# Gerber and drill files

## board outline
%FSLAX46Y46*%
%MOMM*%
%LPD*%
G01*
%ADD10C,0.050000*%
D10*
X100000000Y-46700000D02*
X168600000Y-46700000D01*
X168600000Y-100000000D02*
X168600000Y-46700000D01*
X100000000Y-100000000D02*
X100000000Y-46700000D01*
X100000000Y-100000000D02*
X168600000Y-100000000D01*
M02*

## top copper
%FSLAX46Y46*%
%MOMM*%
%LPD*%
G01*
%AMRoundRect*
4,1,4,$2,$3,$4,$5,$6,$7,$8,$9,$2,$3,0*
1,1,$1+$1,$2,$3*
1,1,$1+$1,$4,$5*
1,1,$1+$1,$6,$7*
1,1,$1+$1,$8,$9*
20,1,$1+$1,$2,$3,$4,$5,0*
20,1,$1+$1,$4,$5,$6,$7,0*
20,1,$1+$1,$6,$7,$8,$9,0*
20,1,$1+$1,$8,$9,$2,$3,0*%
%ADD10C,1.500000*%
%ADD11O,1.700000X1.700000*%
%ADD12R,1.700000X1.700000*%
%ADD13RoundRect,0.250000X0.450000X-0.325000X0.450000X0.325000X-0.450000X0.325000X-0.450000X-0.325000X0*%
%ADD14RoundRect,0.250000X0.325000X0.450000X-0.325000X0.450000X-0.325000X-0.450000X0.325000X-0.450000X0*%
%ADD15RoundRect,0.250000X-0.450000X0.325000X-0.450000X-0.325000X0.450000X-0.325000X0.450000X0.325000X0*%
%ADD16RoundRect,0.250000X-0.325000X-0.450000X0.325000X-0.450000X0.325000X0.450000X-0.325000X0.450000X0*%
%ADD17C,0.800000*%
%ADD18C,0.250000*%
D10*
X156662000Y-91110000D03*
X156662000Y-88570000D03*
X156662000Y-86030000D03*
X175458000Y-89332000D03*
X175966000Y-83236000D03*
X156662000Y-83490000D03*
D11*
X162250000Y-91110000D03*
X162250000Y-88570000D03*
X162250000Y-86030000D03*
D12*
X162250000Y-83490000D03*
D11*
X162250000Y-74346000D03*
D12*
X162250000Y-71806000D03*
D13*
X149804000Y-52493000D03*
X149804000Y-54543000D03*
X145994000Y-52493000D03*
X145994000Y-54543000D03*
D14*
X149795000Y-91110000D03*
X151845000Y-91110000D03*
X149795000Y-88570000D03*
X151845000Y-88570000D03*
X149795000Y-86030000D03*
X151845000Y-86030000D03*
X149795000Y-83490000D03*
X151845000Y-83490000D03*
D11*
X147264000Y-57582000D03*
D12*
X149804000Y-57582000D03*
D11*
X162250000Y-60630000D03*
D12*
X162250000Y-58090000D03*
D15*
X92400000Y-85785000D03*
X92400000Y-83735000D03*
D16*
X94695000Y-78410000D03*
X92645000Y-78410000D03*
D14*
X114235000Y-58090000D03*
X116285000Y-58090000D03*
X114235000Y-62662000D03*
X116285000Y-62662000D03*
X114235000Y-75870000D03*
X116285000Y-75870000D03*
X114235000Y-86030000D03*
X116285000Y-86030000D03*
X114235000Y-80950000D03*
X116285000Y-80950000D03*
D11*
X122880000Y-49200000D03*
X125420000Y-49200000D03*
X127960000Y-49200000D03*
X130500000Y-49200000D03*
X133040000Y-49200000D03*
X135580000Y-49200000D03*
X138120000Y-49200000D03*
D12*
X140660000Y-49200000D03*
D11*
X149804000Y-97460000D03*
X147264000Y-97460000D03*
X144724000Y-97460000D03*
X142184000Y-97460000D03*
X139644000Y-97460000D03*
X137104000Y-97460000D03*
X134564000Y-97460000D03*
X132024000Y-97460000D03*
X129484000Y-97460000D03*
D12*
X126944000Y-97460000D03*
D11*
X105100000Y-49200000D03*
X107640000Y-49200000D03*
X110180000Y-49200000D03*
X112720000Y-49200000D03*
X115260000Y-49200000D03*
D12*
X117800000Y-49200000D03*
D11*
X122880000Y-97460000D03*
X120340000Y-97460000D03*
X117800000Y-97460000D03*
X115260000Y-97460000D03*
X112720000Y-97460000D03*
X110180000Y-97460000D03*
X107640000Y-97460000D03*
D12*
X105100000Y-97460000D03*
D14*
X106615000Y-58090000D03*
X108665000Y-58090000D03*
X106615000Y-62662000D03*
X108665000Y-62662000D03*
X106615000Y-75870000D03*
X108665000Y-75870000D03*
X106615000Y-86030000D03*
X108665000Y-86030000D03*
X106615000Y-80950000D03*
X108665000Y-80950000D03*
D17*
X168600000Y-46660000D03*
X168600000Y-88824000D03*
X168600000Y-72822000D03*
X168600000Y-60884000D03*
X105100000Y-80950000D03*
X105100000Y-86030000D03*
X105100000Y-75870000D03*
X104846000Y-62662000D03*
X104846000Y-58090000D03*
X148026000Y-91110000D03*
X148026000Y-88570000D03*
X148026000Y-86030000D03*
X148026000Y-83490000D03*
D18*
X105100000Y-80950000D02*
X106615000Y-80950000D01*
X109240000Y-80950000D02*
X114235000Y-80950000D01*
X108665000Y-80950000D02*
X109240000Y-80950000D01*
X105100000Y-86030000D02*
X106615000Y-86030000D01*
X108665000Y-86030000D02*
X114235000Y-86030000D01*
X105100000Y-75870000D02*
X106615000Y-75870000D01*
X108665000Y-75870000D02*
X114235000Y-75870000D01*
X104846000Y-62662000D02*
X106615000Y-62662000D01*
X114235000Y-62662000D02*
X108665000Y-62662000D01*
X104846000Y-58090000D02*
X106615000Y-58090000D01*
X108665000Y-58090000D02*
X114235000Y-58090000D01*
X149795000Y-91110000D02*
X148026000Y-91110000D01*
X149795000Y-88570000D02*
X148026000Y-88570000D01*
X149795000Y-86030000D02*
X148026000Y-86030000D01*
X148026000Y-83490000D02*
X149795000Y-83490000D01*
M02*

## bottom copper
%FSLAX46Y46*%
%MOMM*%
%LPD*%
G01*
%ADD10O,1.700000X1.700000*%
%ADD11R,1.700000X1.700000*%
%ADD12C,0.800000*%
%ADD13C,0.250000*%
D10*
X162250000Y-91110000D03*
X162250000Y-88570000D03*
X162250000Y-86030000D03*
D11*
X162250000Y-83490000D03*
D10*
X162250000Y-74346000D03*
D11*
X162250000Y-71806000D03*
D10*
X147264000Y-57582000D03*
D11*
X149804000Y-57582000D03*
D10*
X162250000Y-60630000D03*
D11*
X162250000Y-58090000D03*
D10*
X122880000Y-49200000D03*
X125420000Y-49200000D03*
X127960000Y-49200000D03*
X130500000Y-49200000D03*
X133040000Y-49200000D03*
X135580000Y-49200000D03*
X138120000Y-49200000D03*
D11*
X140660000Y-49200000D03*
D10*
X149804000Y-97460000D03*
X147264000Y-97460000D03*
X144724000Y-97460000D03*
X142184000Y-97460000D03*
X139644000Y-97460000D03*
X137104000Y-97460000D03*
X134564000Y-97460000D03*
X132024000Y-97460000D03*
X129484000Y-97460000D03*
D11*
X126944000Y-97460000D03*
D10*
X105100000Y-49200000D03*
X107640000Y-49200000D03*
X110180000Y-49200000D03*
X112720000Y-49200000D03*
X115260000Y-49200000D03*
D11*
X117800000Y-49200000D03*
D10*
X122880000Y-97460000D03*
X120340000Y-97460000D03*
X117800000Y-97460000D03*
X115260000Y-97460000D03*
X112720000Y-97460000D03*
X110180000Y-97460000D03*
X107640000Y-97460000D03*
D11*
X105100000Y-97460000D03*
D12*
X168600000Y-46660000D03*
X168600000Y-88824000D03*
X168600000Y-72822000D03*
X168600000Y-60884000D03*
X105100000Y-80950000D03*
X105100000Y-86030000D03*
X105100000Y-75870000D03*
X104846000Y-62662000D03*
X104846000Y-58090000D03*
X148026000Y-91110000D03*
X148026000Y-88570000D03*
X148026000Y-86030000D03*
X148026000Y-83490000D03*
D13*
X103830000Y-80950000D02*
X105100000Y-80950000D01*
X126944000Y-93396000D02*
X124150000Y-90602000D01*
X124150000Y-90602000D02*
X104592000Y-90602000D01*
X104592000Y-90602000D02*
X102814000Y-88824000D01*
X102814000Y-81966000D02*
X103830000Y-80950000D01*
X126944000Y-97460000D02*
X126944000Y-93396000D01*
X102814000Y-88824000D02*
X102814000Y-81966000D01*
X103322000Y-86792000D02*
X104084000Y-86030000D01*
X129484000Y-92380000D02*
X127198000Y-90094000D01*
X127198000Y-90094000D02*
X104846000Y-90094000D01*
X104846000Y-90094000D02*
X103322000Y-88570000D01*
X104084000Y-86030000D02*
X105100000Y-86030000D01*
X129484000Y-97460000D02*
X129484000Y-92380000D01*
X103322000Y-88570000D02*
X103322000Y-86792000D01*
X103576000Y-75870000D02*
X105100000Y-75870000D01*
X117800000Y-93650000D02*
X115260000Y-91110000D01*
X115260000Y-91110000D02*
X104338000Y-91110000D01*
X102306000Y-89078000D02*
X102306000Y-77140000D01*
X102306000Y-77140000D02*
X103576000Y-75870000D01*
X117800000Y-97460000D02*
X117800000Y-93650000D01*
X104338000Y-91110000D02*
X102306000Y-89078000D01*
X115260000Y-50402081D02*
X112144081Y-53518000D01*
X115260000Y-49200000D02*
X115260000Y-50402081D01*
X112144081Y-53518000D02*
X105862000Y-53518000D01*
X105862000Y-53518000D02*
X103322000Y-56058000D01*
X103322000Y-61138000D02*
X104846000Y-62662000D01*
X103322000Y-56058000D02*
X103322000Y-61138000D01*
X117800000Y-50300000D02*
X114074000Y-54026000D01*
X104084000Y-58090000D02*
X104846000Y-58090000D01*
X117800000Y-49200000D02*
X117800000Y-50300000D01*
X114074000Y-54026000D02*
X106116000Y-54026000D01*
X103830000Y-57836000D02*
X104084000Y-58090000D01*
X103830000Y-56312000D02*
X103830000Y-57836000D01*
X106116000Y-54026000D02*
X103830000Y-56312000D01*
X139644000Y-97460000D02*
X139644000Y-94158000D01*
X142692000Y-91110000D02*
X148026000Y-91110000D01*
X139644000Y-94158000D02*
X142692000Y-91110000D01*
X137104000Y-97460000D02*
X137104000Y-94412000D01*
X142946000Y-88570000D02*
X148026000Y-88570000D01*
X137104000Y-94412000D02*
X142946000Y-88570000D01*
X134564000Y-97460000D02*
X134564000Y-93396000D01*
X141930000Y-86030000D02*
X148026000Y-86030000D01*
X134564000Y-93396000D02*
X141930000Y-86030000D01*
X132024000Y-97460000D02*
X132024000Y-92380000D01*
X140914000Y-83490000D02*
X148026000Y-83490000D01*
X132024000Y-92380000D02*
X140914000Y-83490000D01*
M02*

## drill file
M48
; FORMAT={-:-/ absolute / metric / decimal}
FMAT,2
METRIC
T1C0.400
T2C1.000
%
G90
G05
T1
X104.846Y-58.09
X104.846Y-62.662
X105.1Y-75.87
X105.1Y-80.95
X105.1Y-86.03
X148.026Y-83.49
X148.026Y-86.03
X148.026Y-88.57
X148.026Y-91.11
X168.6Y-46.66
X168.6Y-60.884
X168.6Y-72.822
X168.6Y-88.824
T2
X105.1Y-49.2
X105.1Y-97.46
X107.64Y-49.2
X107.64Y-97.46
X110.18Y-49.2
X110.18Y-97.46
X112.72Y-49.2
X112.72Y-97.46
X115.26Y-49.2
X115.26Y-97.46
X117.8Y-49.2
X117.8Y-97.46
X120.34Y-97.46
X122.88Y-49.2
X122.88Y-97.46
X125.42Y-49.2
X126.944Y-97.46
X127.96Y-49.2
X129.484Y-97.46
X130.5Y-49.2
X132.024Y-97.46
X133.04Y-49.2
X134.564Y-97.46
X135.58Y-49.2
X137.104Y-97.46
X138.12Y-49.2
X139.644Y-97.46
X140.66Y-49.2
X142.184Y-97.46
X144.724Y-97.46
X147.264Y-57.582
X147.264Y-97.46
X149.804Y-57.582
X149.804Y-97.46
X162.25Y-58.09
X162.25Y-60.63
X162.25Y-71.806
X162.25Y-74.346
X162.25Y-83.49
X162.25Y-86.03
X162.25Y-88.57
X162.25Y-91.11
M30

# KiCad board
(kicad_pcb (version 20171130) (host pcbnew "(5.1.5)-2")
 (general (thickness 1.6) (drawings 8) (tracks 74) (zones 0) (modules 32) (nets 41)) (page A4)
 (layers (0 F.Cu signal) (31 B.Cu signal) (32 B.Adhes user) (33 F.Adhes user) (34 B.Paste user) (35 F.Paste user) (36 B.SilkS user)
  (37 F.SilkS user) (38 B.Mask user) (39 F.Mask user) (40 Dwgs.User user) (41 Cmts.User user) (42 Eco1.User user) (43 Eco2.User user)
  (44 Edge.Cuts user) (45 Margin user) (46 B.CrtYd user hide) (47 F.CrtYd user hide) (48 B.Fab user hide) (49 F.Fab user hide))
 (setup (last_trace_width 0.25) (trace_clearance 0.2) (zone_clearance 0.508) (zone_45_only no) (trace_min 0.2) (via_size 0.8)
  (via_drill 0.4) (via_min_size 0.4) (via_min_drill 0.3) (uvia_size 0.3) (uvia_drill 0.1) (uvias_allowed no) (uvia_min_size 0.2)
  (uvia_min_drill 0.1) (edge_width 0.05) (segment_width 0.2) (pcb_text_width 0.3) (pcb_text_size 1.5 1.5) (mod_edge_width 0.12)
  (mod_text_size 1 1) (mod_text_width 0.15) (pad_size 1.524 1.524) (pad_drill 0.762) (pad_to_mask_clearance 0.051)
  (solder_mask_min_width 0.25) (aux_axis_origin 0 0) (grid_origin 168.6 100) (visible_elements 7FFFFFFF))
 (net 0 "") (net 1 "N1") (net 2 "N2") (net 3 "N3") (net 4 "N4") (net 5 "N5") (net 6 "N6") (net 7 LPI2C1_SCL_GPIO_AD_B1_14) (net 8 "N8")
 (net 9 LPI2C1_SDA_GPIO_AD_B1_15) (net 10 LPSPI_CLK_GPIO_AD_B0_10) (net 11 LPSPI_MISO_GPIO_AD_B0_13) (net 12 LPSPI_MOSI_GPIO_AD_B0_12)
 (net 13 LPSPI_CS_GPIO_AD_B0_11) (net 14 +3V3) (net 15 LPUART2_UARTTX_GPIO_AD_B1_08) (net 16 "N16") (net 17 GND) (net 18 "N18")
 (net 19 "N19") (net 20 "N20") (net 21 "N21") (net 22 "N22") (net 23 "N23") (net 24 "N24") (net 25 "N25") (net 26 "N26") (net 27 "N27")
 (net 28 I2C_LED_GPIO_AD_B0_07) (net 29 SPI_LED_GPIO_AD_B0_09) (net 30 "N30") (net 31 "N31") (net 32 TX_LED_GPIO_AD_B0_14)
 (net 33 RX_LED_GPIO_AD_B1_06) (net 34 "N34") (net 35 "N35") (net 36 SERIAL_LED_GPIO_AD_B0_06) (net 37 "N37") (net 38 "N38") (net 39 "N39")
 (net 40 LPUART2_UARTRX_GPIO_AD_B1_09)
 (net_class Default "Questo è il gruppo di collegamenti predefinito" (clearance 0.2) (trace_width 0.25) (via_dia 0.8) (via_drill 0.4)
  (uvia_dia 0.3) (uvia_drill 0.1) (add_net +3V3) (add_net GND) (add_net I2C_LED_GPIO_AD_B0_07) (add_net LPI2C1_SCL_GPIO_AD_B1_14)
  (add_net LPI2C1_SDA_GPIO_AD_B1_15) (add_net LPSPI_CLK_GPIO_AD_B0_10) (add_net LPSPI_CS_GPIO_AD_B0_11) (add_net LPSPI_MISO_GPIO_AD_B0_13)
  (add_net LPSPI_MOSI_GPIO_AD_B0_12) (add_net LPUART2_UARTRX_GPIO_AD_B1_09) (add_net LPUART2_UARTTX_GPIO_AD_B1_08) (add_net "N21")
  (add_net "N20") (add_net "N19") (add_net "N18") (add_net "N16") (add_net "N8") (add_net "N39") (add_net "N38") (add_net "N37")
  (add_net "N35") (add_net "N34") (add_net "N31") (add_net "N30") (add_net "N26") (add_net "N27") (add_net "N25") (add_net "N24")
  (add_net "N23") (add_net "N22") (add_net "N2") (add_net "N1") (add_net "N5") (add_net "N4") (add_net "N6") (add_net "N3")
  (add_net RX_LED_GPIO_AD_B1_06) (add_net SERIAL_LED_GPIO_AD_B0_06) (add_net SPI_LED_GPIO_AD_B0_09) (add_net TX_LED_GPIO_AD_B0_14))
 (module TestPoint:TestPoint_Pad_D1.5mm (layer F.Cu) (at 156.662 91.11)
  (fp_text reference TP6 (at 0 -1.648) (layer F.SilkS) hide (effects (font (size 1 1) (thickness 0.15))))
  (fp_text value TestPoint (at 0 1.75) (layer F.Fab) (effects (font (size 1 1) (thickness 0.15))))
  (pad 1 smd circle (at 0 0) (size 1.5 1.5) (layers F.Cu F.Mask) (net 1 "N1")))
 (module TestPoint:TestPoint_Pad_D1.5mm (layer F.Cu) (at 156.662 88.57)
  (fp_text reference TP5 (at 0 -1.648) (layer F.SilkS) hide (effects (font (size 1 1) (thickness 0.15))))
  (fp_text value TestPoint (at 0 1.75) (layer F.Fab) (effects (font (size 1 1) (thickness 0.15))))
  (pad 1 smd circle (at 0 0) (size 1.5 1.5) (layers F.Cu F.Mask) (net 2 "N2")))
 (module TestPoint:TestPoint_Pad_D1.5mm (layer F.Cu) (at 156.662 86.03)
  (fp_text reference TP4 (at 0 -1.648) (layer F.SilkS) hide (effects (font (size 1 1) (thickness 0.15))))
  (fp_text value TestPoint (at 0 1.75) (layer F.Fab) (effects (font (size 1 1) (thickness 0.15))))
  (pad 1 smd circle (at 0 0) (size 1.5 1.5) (layers F.Cu F.Mask) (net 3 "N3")))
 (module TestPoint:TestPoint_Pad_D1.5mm (layer F.Cu) (at 175.458 89.332)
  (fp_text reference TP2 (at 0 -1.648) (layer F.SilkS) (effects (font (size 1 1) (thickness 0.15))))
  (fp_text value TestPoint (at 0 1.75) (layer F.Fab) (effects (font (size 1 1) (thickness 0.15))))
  (pad 1 smd circle (at 0 0) (size 1.5 1.5) (layers F.Cu F.Mask) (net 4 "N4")))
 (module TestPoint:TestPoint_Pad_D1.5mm (layer F.Cu) (at 175.966 83.236)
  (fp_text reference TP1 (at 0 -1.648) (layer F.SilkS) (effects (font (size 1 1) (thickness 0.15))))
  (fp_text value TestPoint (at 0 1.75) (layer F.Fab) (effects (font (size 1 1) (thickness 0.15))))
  (pad 1 smd circle (at 0 0) (size 1.5 1.5) (layers F.Cu F.Mask) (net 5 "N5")))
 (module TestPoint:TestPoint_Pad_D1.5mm (layer F.Cu) (at 156.662 83.49)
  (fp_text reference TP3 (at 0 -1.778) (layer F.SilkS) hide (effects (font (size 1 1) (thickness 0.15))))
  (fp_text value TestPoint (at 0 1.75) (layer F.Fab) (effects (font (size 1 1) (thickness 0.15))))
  (pad 1 smd circle (at 0 0) (size 1.5 1.5) (layers F.Cu F.Mask) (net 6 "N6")))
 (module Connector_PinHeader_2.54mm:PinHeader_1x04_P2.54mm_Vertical (layer F.Cu) (at 162.25 83.49)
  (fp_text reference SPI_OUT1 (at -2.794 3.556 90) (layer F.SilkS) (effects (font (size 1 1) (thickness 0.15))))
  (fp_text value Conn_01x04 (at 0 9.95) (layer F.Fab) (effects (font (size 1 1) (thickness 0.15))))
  (pad 4 thru_hole oval (at 0 7.62) (size 1.7 1.7) (drill 1) (layers *.Cu *.Mask) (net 1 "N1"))
  (pad 3 thru_hole oval (at 0 5.08) (size 1.7 1.7) (drill 1) (layers *.Cu *.Mask) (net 2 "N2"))
  (pad 2 thru_hole oval (at 0 2.54) (size 1.7 1.7) (drill 1) (layers *.Cu *.Mask) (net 3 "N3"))
  (pad 1 thru_hole rect (at 0 0) (size 1.7 1.7) (drill 1) (layers *.Cu *.Mask) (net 6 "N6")))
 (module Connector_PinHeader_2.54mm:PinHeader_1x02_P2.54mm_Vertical (layer F.Cu) (at 162.25 71.806)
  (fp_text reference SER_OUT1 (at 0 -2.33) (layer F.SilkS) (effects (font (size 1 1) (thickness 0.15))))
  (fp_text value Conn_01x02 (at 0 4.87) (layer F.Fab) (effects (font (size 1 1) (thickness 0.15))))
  (pad 2 thru_hole oval (at 0 2.54) (size 1.7 1.7) (drill 1) (layers *.Cu *.Mask) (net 4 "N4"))
  (pad 1 thru_hole rect (at 0 0) (size 1.7 1.7) (drill 1) (layers *.Cu *.Mask) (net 5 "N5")))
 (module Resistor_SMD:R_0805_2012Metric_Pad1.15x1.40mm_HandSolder (layer F.Cu) (at 149.804 53.518 90)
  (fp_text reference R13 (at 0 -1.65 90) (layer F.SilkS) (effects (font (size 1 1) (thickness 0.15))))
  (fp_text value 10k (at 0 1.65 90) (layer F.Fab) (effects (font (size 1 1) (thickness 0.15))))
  (pad 2 smd roundrect (at 1.025 0 90) (size 1.15 1.4) (layers F.Cu F.Paste F.Mask) (roundrect_rratio 0.217391)
   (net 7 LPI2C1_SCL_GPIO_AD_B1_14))
  (pad 1 smd roundrect (at -1.025 0 90) (size 1.15 1.4) (layers F.Cu F.Paste F.Mask) (roundrect_rratio 0.217391) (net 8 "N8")))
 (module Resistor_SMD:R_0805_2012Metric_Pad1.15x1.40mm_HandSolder (layer F.Cu) (at 145.994 53.518 90)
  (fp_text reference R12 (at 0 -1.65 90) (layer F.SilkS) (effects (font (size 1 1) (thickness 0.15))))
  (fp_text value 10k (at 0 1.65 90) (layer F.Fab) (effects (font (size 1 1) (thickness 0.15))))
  (pad 2 smd roundrect (at 1.025 0 90) (size 1.15 1.4) (layers F.Cu F.Paste F.Mask) (roundrect_rratio 0.217391)
   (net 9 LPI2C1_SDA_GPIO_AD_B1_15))
  (pad 1 smd roundrect (at -1.025 0 90) (size 1.15 1.4) (layers F.Cu F.Paste F.Mask) (roundrect_rratio 0.217391) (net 8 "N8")))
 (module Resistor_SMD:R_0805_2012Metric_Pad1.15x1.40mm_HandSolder (layer F.Cu) (at 150.82 91.11 180)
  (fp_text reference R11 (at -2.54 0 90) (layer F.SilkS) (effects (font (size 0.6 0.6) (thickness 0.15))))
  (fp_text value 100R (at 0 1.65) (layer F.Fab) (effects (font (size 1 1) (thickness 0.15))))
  (pad 2 smd roundrect (at 1.025 0 180) (size 1.15 1.4) (layers F.Cu F.Paste F.Mask) (roundrect_rratio 0.217391)
   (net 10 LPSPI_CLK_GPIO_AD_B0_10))
  (pad 1 smd roundrect (at -1.025 0 180) (size 1.15 1.4) (layers F.Cu F.Paste F.Mask) (roundrect_rratio 0.217391) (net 1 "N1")))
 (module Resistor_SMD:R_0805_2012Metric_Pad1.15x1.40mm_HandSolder (layer F.Cu) (at 150.82 88.57 180)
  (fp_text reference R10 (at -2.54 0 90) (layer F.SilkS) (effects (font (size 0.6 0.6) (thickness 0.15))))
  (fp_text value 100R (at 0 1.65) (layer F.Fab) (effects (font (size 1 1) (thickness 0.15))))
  (pad 2 smd roundrect (at 1.025 0 180) (size 1.15 1.4) (layers F.Cu F.Paste F.Mask) (roundrect_rratio 0.217391)
   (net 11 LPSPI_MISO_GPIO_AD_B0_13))
  (pad 1 smd roundrect (at -1.025 0 180) (size 1.15 1.4) (layers F.Cu F.Paste F.Mask) (roundrect_rratio 0.217391) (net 2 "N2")))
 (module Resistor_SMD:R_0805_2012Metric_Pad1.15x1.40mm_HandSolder (layer F.Cu) (at 150.82 86.03 180)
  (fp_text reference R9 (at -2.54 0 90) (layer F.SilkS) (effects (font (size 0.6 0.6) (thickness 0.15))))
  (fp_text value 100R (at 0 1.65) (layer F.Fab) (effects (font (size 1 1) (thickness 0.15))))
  (pad 2 smd roundrect (at 1.025 0 180) (size 1.15 1.4) (layers F.Cu F.Paste F.Mask) (roundrect_rratio 0.217391)
   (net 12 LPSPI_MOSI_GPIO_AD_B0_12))
  (pad 1 smd roundrect (at -1.025 0 180) (size 1.15 1.4) (layers F.Cu F.Paste F.Mask) (roundrect_rratio 0.217391) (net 3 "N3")))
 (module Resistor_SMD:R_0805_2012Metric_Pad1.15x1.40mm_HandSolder (layer F.Cu) (at 150.82 83.49 180)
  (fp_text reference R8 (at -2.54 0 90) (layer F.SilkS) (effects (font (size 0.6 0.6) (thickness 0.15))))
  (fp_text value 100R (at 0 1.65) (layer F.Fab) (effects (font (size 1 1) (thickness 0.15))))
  (pad 2 smd roundrect (at 1.025 0 180) (size 1.15 1.4) (layers F.Cu F.Paste F.Mask) (roundrect_rratio 0.217391)
   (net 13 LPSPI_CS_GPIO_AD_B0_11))
  (pad 1 smd roundrect (at -1.025 0 180) (size 1.15 1.4) (layers F.Cu F.Paste F.Mask) (roundrect_rratio 0.217391) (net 6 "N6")))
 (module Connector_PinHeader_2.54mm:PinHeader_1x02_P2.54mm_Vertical (layer F.Cu) (at 149.804 57.582 270)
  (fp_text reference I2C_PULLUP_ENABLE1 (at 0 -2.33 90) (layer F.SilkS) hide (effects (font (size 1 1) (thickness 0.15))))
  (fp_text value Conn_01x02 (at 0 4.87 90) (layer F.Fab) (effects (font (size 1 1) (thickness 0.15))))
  (pad 2 thru_hole oval (at 0 2.54 270) (size 1.7 1.7) (drill 1) (layers *.Cu *.Mask) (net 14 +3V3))
  (pad 1 thru_hole rect (at 0 0 270) (size 1.7 1.7) (drill 1) (layers *.Cu *.Mask) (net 8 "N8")))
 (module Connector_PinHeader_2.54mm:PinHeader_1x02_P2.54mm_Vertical (layer F.Cu) (at 162.25 58.09)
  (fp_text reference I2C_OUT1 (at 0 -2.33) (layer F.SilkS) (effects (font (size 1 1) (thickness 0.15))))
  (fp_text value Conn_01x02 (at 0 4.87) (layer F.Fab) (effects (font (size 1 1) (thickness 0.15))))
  (pad 2 thru_hole oval (at 0 2.54) (size 1.7 1.7) (drill 1) (layers *.Cu *.Mask) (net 7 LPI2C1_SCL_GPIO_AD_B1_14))
  (pad 1 thru_hole rect (at 0 0) (size 1.7 1.7) (drill 1) (layers *.Cu *.Mask) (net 9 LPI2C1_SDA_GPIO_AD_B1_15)))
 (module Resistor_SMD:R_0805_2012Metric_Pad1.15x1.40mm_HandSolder (layer F.Cu) (at 92.4 84.76 270)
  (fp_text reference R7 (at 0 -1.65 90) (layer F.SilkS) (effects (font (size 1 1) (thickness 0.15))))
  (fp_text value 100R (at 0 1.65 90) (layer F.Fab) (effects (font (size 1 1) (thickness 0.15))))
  (pad 2 smd roundrect (at 1.025 0 270) (size 1.15 1.4) (layers F.Cu F.Paste F.Mask) (roundrect_rratio 0.217391)
   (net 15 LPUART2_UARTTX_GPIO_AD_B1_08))
  (pad 1 smd roundrect (at -1.025 0 270) (size 1.15 1.4) (layers F.Cu F.Paste F.Mask) (roundrect_rratio 0.217391) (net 4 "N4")))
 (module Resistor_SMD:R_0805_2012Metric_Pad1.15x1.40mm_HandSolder (layer F.Cu) (at 93.67 78.41)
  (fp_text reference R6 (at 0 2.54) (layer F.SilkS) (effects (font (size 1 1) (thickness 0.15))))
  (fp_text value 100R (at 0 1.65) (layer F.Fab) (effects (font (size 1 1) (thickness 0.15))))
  (pad 2 smd roundrect (at 1.025 0) (size 1.15 1.4) (layers F.Cu F.Paste F.Mask) (roundrect_rratio 0.217391)
   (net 15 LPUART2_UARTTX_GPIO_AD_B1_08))
  (pad 1 smd roundrect (at -1.025 0) (size 1.15 1.4) (layers F.Cu F.Paste F.Mask) (roundrect_rratio 0.217391) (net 5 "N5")))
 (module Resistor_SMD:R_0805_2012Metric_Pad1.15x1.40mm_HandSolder (layer F.Cu) (at 115.26 58.09 180)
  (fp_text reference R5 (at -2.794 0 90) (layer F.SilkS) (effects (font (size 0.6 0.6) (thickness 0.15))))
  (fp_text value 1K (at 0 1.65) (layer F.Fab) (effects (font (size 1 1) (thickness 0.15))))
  (pad 2 smd roundrect (at 1.025 0 180) (size 1.15 1.4) (layers F.Cu F.Paste F.Mask) (roundrect_rratio 0.217391) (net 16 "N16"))
  (pad 1 smd roundrect (at -1.025 0 180) (size 1.15 1.4) (layers F.Cu F.Paste F.Mask) (roundrect_rratio 0.217391) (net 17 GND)))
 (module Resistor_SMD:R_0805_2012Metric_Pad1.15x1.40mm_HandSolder (layer F.Cu) (at 115.26 62.662 180)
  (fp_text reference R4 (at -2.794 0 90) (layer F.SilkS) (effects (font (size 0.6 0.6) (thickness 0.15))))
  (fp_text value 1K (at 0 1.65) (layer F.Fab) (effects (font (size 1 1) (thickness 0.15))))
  (pad 2 smd roundrect (at 1.025 0 180) (size 1.15 1.4) (layers F.Cu F.Paste F.Mask) (roundrect_rratio 0.217391) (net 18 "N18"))
  (pad 1 smd roundrect (at -1.025 0 180) (size 1.15 1.4) (layers F.Cu F.Paste F.Mask) (roundrect_rratio 0.217391) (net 17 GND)))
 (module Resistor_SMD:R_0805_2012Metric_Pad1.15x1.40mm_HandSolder (layer F.Cu) (at 115.26 75.87 180)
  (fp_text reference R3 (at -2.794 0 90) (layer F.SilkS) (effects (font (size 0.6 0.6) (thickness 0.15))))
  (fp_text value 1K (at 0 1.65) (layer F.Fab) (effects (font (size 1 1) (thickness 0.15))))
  (pad 2 smd roundrect (at 1.025 0 180) (size 1.15 1.4) (layers F.Cu F.Paste F.Mask) (roundrect_rratio 0.217391) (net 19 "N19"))
  (pad 1 smd roundrect (at -1.025 0 180) (size 1.15 1.4) (layers F.Cu F.Paste F.Mask) (roundrect_rratio 0.217391) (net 17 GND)))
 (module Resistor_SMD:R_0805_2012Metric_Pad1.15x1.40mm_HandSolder (layer F.Cu) (at 115.26 86.03 180)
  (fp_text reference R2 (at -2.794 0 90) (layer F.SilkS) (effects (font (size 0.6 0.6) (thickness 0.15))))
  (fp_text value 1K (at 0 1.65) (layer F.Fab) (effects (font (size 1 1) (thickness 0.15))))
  (pad 2 smd roundrect (at 1.025 0 180) (size 1.15 1.4) (layers F.Cu F.Paste F.Mask) (roundrect_rratio 0.217391) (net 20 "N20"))
  (pad 1 smd roundrect (at -1.025 0 180) (size 1.15 1.4) (layers F.Cu F.Paste F.Mask) (roundrect_rratio 0.217391) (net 17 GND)))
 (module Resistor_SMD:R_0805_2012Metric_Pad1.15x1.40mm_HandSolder (layer F.Cu) (at 115.26 80.95 180)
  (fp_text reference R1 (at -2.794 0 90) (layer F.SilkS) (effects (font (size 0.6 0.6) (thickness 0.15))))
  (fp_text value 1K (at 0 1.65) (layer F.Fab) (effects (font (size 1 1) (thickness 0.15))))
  (pad 2 smd roundrect (at 1.025 0 180) (size 1.15 1.4) (layers F.Cu F.Paste F.Mask) (roundrect_rratio 0.217391) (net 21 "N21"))
  (pad 1 smd roundrect (at -1.025 0 180) (size 1.15 1.4) (layers F.Cu F.Paste F.Mask) (roundrect_rratio 0.217391) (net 17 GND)))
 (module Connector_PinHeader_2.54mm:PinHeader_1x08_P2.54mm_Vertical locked (layer F.Cu) (at 140.66 49.2 270)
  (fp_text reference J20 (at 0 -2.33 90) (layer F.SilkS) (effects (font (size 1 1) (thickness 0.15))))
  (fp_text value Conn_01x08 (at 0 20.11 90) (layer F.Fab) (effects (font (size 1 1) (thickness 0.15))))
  (pad 8 thru_hole oval (at 0 17.78 270) (size 1.7 1.7) (drill 1) (layers *.Cu *.Mask) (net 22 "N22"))
  (pad 7 thru_hole oval (at 0 15.24 270) (size 1.7 1.7) (drill 1) (layers *.Cu *.Mask) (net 17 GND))
  (pad 6 thru_hole oval (at 0 12.7 270) (size 1.7 1.7) (drill 1) (layers *.Cu *.Mask) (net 17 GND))
  (pad 5 thru_hole oval (at 0 10.16 270) (size 1.7 1.7) (drill 1) (layers *.Cu *.Mask) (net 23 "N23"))
  (pad 4 thru_hole oval (at 0 7.62 270) (size 1.7 1.7) (drill 1) (layers *.Cu *.Mask) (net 14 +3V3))
  (pad 3 thru_hole oval (at 0 5.08 270) (size 1.7 1.7) (drill 1) (layers *.Cu *.Mask) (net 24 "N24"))
  (pad 2 thru_hole oval (at 0 2.54 270) (size 1.7 1.7) (drill 1) (layers *.Cu *.Mask) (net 14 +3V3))
  (pad 1 thru_hole rect (at 0 0 270) (size 1.7 1.7) (drill 1) (layers *.Cu *.Mask) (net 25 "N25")))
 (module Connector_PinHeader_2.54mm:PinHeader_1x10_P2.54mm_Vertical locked (layer F.Cu) (at 126.944 97.46 90)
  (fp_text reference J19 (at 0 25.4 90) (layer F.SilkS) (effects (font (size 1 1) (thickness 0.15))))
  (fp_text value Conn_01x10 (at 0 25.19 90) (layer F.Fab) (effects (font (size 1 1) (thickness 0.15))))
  (pad 10 thru_hole oval (at 0 22.86 90) (size 1.7 1.7) (drill 1) (layers *.Cu *.Mask) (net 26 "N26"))
  (pad 9 thru_hole oval (at 0 20.32 90) (size 1.7 1.7) (drill 1) (layers *.Cu *.Mask) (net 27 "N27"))
  (pad 8 thru_hole oval (at 0 17.78 90) (size 1.7 1.7) (drill 1) (layers *.Cu *.Mask) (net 14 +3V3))
  (pad 7 thru_hole oval (at 0 15.24 90) (size 1.7 1.7) (drill 1) (layers *.Cu *.Mask) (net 17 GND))
  (pad 6 thru_hole oval (at 0 12.7 90) (size 1.7 1.7) (drill 1) (layers *.Cu *.Mask) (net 10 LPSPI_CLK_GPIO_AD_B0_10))
  (pad 5 thru_hole oval (at 0 10.16 90) (size 1.7 1.7) (drill 1) (layers *.Cu *.Mask) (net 11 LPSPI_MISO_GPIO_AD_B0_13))
  (pad 4 thru_hole oval (at 0 7.62 90) (size 1.7 1.7) (drill 1) (layers *.Cu *.Mask) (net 12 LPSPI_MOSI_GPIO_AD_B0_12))
  (pad 3 thru_hole oval (at 0 5.08 90) (size 1.7 1.7) (drill 1) (layers *.Cu *.Mask) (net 13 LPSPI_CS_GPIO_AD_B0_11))
  (pad 2 thru_hole oval (at 0 2.54 90) (size 1.7 1.7) (drill 1) (layers *.Cu *.Mask) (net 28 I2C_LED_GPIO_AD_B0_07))
  (pad 1 thru_hole rect (at 0 0 90) (size 1.7 1.7) (drill 1) (layers *.Cu *.Mask) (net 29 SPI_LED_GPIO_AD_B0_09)))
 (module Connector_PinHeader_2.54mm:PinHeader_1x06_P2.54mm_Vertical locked (layer F.Cu) (at 117.8 49.2 270)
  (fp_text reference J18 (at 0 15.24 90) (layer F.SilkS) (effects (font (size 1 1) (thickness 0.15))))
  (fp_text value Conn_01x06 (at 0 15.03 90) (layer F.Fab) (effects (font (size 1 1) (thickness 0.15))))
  (pad 6 thru_hole oval (at 0 12.7 270) (size 1.7 1.7) (drill 1) (layers *.Cu *.Mask) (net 7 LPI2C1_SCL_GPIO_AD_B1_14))
  (pad 5 thru_hole oval (at 0 10.16 270) (size 1.7 1.7) (drill 1) (layers *.Cu *.Mask) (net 9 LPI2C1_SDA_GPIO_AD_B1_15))
  (pad 4 thru_hole oval (at 0 7.62 270) (size 1.7 1.7) (drill 1) (layers *.Cu *.Mask) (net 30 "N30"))
  (pad 3 thru_hole oval (at 0 5.08 270) (size 1.7 1.7) (drill 1) (layers *.Cu *.Mask) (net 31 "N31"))
  (pad 2 thru_hole oval (at 0 2.54 270) (size 1.7 1.7) (drill 1) (layers *.Cu *.Mask) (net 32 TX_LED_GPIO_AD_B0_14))
  (pad 1 thru_hole rect (at 0 0 270) (size 1.7 1.7) (drill 1) (layers *.Cu *.Mask) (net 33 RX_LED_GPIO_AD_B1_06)))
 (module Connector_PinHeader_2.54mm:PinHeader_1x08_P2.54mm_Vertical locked (layer F.Cu) (at 105.1 97.46 90)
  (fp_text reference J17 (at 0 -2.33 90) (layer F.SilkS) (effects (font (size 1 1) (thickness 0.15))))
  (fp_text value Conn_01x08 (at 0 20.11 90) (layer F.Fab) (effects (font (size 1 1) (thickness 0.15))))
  (pad 8 thru_hole oval (at 0 17.78 90) (size 1.7 1.7) (drill 1) (layers *.Cu *.Mask) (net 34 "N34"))
  (pad 7 thru_hole oval (at 0 15.24 90) (size 1.7 1.7) (drill 1) (layers *.Cu *.Mask) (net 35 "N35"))
  (pad 6 thru_hole oval (at 0 12.7 90) (size 1.7 1.7) (drill 1) (layers *.Cu *.Mask) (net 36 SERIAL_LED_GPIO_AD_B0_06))
  (pad 5 thru_hole oval (at 0 10.16 90) (size 1.7 1.7) (drill 1) (layers *.Cu *.Mask) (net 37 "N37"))
  (pad 4 thru_hole oval (at 0 7.62 90) (size 1.7 1.7) (drill 1) (layers *.Cu *.Mask) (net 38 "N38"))
  (pad 3 thru_hole oval (at 0 5.08 90) (size 1.7 1.7) (drill 1) (layers *.Cu *.Mask) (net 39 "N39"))
  (pad 2 thru_hole oval (at 0 2.54 90) (size 1.7 1.7) (drill 1) (layers *.Cu *.Mask) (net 15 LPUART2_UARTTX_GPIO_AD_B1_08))
  (pad 1 thru_hole rect (at 0 0 90) (size 1.7 1.7) (drill 1) (layers *.Cu *.Mask) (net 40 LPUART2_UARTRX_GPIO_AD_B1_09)))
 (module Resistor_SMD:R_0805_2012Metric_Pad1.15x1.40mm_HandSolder (layer F.Cu) (at 107.64 58.09 180)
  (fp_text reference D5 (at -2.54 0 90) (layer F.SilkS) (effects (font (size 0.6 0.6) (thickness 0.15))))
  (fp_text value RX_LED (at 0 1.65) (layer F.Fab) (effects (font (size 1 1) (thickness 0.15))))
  (pad 2 smd roundrect (at 1.025 0 180) (size 1.15 1.4) (layers F.Cu F.Paste F.Mask) (roundrect_rratio 0.217391)
   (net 33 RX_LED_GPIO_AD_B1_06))
  (pad 1 smd roundrect (at -1.025 0 180) (size 1.15 1.4) (layers F.Cu F.Paste F.Mask) (roundrect_rratio 0.217391) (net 16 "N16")))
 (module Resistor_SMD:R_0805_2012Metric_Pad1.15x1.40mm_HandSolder (layer F.Cu) (at 107.64 62.662 180)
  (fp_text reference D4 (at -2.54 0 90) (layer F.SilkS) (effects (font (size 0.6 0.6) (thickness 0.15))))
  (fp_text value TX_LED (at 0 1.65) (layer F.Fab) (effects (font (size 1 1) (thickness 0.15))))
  (pad 2 smd roundrect (at 1.025 0 180) (size 1.15 1.4) (layers F.Cu F.Paste F.Mask) (roundrect_rratio 0.217391)
   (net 32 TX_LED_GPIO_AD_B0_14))
  (pad 1 smd roundrect (at -1.025 0 180) (size 1.15 1.4) (layers F.Cu F.Paste F.Mask) (roundrect_rratio 0.217391) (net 18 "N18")))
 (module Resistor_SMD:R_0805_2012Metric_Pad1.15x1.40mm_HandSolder (layer F.Cu) (at 107.64 75.87 180)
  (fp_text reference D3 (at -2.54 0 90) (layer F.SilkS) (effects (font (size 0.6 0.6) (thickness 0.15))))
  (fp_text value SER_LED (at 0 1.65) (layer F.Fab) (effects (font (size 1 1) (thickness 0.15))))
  (pad 2 smd roundrect (at 1.025 0 180) (size 1.15 1.4) (layers F.Cu F.Paste F.Mask) (roundrect_rratio 0.217391)
   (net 36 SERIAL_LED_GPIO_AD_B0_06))
  (pad 1 smd roundrect (at -1.025 0 180) (size 1.15 1.4) (layers F.Cu F.Paste F.Mask) (roundrect_rratio 0.217391) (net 19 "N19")))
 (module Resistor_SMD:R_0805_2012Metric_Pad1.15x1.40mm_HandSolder (layer F.Cu) (at 107.64 86.03 180)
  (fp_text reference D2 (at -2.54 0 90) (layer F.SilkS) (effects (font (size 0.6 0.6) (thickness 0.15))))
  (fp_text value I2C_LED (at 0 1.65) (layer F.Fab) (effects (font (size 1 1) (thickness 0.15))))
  (pad 2 smd roundrect (at 1.025 0 180) (size 1.15 1.4) (layers F.Cu F.Paste F.Mask) (roundrect_rratio 0.217391)
   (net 28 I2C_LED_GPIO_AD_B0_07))
  (pad 1 smd roundrect (at -1.025 0 180) (size 1.15 1.4) (layers F.Cu F.Paste F.Mask) (roundrect_rratio 0.217391) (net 20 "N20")))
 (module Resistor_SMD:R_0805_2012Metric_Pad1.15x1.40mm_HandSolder (layer F.Cu) (at 107.64 80.95 180)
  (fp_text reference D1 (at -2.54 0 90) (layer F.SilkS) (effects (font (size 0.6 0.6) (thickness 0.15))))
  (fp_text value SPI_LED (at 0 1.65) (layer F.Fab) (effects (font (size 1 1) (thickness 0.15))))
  (pad 2 smd roundrect (at 1.025 0 180) (size 1.15 1.4) (layers F.Cu F.Paste F.Mask) (roundrect_rratio 0.217391)
   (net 29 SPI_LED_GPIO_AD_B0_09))
  (pad 1 smd roundrect (at -1.025 0 180) (size 1.15 1.4) (layers F.Cu F.Paste F.Mask) (roundrect_rratio 0.217391) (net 21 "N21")))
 (gr_line (start 100 46.7) (end 168.6 46.7) (layer Edge.Cuts) (width 0.05))
 (gr_line (start 168.6 100) (end 168.6 46.7) (layer Edge.Cuts) (width 0.05))
 (gr_line (start 100 100) (end 100 46.7) (layer Edge.Cuts) (width 0.05))
 (gr_line (start 100 100) (end 168.6 100) (layer Edge.Cuts) (width 0.05))
 (via (at 168.6 46.66) (size 0.8) (drill 0.4) (layers F.Cu B.Cu) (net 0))
 (via (at 168.6 88.824) (size 0.8) (drill 0.4) (layers F.Cu B.Cu) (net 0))
 (via (at 168.6 72.822) (size 0.8) (drill 0.4) (layers F.Cu B.Cu) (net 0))
 (via (at 168.6 60.884) (size 0.8) (drill 0.4) (layers F.Cu B.Cu) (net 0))
 (via (at 105.1 80.95) (size 0.8) (drill 0.4) (layers F.Cu B.Cu) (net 29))
 (segment (start 103.83 80.95) (end 105.1 80.95) (width 0.25) (layer B.Cu) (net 29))
 (segment (start 126.944 93.396) (end 124.15 90.602) (width 0.25) (layer B.Cu) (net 29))
 (segment (start 124.15 90.602) (end 104.592 90.602) (width 0.25) (layer B.Cu) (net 29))
 (segment (start 104.592 90.602) (end 102.814 88.824) (width 0.25) (layer B.Cu) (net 29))
 (segment (start 102.814 81.966) (end 103.83 80.95) (width 0.25) (layer B.Cu) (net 29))
 (segment (start 126.944 97.46) (end 126.944 93.396) (width 0.25) (layer B.Cu) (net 29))
 (segment (start 102.814 88.824) (end 102.814 81.966) (width 0.25) (layer B.Cu) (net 29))
 (segment (start 105.1 80.95) (end 106.615 80.95) (width 0.25) (layer F.Cu) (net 29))
 (segment (start 109.24 80.95) (end 114.235 80.95) (width 0.25) (layer F.Cu) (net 21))
 (segment (start 108.665 80.95) (end 109.24 80.95) (width 0.25) (layer F.Cu) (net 21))
 (via (at 105.1 86.03) (size 0.8) (drill 0.4) (layers F.Cu B.Cu) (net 28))
 (segment (start 103.322 86.792) (end 104.084 86.03) (width 0.25) (layer B.Cu) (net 28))
 (segment (start 129.484 92.38) (end 127.198 90.094) (width 0.25) (layer B.Cu) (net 28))
 (segment (start 127.198 90.094) (end 104.846 90.094) (width 0.25) (layer B.Cu) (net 28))
 (segment (start 104.846 90.094) (end 103.322 88.57) (width 0.25) (layer B.Cu) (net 28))
 (segment (start 104.084 86.03) (end 105.1 86.03) (width 0.25) (layer B.Cu) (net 28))
 (segment (start 129.484 97.46) (end 129.484 92.38) (width 0.25) (layer B.Cu) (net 28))
 (segment (start 103.322 88.57) (end 103.322 86.792) (width 0.25) (layer B.Cu) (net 28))
 (segment (start 105.1 86.03) (end 106.615 86.03) (width 0.25) (layer F.Cu) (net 28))
 (segment (start 108.665 86.03) (end 114.235 86.03) (width 0.25) (layer F.Cu) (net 20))
 (via (at 105.1 75.87) (size 0.8) (drill 0.4) (layers F.Cu B.Cu) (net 36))
 (segment (start 103.576 75.87) (end 105.1 75.87) (width 0.25) (layer B.Cu) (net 36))
 (segment (start 117.8 93.65) (end 115.26 91.11) (width 0.25) (layer B.Cu) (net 36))
 (segment (start 115.26 91.11) (end 104.338 91.11) (width 0.25) (layer B.Cu) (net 36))
 (segment (start 102.306 89.078) (end 102.306 77.14) (width 0.25) (layer B.Cu) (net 36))
 (segment (start 102.306 77.14) (end 103.576 75.87) (width 0.25) (layer B.Cu) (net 36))
 (segment (start 117.8 97.46) (end 117.8 93.65) (width 0.25) (layer B.Cu) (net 36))
 (segment (start 104.338 91.11) (end 102.306 89.078) (width 0.25) (layer B.Cu) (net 36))
 (segment (start 105.1 75.87) (end 106.615 75.87) (width 0.25) (layer F.Cu) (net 36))
 (segment (start 108.665 75.87) (end 114.235 75.87) (width 0.25) (layer F.Cu) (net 19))
 (via (at 104.846 62.662) (size 0.8) (drill 0.4) (layers F.Cu B.Cu) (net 32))
 (segment (start 115.26 50.402081) (end 112.144081 53.518) (width 0.25) (layer B.Cu) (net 32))
 (segment (start 115.26 49.2) (end 115.26 50.402081) (width 0.25) (layer B.Cu) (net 32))
 (segment (start 112.144081 53.518) (end 105.862 53.518) (width 0.25) (layer B.Cu) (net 32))
 (segment (start 105.862 53.518) (end 103.322 56.058) (width 0.25) (layer B.Cu) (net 32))
 (segment (start 103.322 61.138) (end 104.846 62.662) (width 0.25) (layer B.Cu) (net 32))
 (segment (start 103.322 56.058) (end 103.322 61.138) (width 0.25) (layer B.Cu) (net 32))
 (segment (start 104.846 62.662) (end 106.615 62.662) (width 0.25) (layer F.Cu) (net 32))
 (segment (start 114.235 62.662) (end 108.665 62.662) (width 0.25) (layer F.Cu) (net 18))
 (via (at 104.846 58.09) (size 0.8) (drill 0.4) (layers F.Cu B.Cu) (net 33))
 (segment (start 117.8 50.3) (end 114.074 54.026) (width 0.25) (layer B.Cu) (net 33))
 (segment (start 104.084 58.09) (end 104.846 58.09) (width 0.25) (layer B.Cu) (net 33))
 (segment (start 117.8 49.2) (end 117.8 50.3) (width 0.25) (layer B.Cu) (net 33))
 (segment (start 114.074 54.026) (end 106.116 54.026) (width 0.25) (layer B.Cu) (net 33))
 (segment (start 103.83 57.836) (end 104.084 58.09) (width 0.25) (layer B.Cu) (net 33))
 (segment (start 103.83 56.312) (end 103.83 57.836) (width 0.25) (layer B.Cu) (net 33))
 (segment (start 106.116 54.026) (end 103.83 56.312) (width 0.25) (layer B.Cu) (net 33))
 (segment (start 104.846 58.09) (end 106.615 58.09) (width 0.25) (layer F.Cu) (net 33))
 (segment (start 108.665 58.09) (end 114.235 58.09) (width 0.25) (layer F.Cu) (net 16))
 (via (at 148.026 91.11) (size 0.8) (drill 0.4) (layers F.Cu B.Cu) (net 10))
 (segment (start 139.644 97.46) (end 139.644 94.158) (width 0.25) (layer B.Cu) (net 10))
 (segment (start 142.692 91.11) (end 148.026 91.11) (width 0.25) (layer B.Cu) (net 10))
 (segment (start 139.644 94.158) (end 142.692 91.11) (width 0.25) (layer B.Cu) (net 10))
 (segment (start 149.795 91.11) (end 148.026 91.11) (width 0.25) (layer F.Cu) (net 10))
 (via (at 148.026 88.57) (size 0.8) (drill 0.4) (layers F.Cu B.Cu) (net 11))
 (segment (start 137.104 97.46) (end 137.104 94.412) (width 0.25) (layer B.Cu) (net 11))
 (segment (start 142.946 88.57) (end 148.026 88.57) (width 0.25) (layer B.Cu) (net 11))
 (segment (start 137.104 94.412) (end 142.946 88.57) (width 0.25) (layer B.Cu) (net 11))
 (segment (start 149.795 88.57) (end 148.026 88.57) (width 0.25) (layer F.Cu) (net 11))
 (via (at 148.026 86.03) (size 0.8) (drill 0.4) (layers F.Cu B.Cu) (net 12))
 (segment (start 134.564 97.46) (end 134.564 93.396) (width 0.25) (layer B.Cu) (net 12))
 (segment (start 141.93 86.03) (end 148.026 86.03) (width 0.25) (layer B.Cu) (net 12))
 (segment (start 134.564 93.396) (end 141.93 86.03) (width 0.25) (layer B.Cu) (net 12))
 (segment (start 149.795 86.03) (end 148.026 86.03) (width 0.25) (layer F.Cu) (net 12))
 (via (at 148.026 83.49) (size 0.8) (drill 0.4) (layers F.Cu B.Cu) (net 13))
 (segment (start 132.024 97.46) (end 132.024 92.38) (width 0.25) (layer B.Cu) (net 13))
 (segment (start 140.914 83.49) (end 148.026 83.49) (width 0.25) (layer B.Cu) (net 13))
 (segment (start 132.024 92.38) (end 140.914 83.49) (width 0.25) (layer B.Cu) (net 13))
 (segment (start 148.026 83.49) (end 149.795 83.49) (width 0.25) (layer F.Cu) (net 13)))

